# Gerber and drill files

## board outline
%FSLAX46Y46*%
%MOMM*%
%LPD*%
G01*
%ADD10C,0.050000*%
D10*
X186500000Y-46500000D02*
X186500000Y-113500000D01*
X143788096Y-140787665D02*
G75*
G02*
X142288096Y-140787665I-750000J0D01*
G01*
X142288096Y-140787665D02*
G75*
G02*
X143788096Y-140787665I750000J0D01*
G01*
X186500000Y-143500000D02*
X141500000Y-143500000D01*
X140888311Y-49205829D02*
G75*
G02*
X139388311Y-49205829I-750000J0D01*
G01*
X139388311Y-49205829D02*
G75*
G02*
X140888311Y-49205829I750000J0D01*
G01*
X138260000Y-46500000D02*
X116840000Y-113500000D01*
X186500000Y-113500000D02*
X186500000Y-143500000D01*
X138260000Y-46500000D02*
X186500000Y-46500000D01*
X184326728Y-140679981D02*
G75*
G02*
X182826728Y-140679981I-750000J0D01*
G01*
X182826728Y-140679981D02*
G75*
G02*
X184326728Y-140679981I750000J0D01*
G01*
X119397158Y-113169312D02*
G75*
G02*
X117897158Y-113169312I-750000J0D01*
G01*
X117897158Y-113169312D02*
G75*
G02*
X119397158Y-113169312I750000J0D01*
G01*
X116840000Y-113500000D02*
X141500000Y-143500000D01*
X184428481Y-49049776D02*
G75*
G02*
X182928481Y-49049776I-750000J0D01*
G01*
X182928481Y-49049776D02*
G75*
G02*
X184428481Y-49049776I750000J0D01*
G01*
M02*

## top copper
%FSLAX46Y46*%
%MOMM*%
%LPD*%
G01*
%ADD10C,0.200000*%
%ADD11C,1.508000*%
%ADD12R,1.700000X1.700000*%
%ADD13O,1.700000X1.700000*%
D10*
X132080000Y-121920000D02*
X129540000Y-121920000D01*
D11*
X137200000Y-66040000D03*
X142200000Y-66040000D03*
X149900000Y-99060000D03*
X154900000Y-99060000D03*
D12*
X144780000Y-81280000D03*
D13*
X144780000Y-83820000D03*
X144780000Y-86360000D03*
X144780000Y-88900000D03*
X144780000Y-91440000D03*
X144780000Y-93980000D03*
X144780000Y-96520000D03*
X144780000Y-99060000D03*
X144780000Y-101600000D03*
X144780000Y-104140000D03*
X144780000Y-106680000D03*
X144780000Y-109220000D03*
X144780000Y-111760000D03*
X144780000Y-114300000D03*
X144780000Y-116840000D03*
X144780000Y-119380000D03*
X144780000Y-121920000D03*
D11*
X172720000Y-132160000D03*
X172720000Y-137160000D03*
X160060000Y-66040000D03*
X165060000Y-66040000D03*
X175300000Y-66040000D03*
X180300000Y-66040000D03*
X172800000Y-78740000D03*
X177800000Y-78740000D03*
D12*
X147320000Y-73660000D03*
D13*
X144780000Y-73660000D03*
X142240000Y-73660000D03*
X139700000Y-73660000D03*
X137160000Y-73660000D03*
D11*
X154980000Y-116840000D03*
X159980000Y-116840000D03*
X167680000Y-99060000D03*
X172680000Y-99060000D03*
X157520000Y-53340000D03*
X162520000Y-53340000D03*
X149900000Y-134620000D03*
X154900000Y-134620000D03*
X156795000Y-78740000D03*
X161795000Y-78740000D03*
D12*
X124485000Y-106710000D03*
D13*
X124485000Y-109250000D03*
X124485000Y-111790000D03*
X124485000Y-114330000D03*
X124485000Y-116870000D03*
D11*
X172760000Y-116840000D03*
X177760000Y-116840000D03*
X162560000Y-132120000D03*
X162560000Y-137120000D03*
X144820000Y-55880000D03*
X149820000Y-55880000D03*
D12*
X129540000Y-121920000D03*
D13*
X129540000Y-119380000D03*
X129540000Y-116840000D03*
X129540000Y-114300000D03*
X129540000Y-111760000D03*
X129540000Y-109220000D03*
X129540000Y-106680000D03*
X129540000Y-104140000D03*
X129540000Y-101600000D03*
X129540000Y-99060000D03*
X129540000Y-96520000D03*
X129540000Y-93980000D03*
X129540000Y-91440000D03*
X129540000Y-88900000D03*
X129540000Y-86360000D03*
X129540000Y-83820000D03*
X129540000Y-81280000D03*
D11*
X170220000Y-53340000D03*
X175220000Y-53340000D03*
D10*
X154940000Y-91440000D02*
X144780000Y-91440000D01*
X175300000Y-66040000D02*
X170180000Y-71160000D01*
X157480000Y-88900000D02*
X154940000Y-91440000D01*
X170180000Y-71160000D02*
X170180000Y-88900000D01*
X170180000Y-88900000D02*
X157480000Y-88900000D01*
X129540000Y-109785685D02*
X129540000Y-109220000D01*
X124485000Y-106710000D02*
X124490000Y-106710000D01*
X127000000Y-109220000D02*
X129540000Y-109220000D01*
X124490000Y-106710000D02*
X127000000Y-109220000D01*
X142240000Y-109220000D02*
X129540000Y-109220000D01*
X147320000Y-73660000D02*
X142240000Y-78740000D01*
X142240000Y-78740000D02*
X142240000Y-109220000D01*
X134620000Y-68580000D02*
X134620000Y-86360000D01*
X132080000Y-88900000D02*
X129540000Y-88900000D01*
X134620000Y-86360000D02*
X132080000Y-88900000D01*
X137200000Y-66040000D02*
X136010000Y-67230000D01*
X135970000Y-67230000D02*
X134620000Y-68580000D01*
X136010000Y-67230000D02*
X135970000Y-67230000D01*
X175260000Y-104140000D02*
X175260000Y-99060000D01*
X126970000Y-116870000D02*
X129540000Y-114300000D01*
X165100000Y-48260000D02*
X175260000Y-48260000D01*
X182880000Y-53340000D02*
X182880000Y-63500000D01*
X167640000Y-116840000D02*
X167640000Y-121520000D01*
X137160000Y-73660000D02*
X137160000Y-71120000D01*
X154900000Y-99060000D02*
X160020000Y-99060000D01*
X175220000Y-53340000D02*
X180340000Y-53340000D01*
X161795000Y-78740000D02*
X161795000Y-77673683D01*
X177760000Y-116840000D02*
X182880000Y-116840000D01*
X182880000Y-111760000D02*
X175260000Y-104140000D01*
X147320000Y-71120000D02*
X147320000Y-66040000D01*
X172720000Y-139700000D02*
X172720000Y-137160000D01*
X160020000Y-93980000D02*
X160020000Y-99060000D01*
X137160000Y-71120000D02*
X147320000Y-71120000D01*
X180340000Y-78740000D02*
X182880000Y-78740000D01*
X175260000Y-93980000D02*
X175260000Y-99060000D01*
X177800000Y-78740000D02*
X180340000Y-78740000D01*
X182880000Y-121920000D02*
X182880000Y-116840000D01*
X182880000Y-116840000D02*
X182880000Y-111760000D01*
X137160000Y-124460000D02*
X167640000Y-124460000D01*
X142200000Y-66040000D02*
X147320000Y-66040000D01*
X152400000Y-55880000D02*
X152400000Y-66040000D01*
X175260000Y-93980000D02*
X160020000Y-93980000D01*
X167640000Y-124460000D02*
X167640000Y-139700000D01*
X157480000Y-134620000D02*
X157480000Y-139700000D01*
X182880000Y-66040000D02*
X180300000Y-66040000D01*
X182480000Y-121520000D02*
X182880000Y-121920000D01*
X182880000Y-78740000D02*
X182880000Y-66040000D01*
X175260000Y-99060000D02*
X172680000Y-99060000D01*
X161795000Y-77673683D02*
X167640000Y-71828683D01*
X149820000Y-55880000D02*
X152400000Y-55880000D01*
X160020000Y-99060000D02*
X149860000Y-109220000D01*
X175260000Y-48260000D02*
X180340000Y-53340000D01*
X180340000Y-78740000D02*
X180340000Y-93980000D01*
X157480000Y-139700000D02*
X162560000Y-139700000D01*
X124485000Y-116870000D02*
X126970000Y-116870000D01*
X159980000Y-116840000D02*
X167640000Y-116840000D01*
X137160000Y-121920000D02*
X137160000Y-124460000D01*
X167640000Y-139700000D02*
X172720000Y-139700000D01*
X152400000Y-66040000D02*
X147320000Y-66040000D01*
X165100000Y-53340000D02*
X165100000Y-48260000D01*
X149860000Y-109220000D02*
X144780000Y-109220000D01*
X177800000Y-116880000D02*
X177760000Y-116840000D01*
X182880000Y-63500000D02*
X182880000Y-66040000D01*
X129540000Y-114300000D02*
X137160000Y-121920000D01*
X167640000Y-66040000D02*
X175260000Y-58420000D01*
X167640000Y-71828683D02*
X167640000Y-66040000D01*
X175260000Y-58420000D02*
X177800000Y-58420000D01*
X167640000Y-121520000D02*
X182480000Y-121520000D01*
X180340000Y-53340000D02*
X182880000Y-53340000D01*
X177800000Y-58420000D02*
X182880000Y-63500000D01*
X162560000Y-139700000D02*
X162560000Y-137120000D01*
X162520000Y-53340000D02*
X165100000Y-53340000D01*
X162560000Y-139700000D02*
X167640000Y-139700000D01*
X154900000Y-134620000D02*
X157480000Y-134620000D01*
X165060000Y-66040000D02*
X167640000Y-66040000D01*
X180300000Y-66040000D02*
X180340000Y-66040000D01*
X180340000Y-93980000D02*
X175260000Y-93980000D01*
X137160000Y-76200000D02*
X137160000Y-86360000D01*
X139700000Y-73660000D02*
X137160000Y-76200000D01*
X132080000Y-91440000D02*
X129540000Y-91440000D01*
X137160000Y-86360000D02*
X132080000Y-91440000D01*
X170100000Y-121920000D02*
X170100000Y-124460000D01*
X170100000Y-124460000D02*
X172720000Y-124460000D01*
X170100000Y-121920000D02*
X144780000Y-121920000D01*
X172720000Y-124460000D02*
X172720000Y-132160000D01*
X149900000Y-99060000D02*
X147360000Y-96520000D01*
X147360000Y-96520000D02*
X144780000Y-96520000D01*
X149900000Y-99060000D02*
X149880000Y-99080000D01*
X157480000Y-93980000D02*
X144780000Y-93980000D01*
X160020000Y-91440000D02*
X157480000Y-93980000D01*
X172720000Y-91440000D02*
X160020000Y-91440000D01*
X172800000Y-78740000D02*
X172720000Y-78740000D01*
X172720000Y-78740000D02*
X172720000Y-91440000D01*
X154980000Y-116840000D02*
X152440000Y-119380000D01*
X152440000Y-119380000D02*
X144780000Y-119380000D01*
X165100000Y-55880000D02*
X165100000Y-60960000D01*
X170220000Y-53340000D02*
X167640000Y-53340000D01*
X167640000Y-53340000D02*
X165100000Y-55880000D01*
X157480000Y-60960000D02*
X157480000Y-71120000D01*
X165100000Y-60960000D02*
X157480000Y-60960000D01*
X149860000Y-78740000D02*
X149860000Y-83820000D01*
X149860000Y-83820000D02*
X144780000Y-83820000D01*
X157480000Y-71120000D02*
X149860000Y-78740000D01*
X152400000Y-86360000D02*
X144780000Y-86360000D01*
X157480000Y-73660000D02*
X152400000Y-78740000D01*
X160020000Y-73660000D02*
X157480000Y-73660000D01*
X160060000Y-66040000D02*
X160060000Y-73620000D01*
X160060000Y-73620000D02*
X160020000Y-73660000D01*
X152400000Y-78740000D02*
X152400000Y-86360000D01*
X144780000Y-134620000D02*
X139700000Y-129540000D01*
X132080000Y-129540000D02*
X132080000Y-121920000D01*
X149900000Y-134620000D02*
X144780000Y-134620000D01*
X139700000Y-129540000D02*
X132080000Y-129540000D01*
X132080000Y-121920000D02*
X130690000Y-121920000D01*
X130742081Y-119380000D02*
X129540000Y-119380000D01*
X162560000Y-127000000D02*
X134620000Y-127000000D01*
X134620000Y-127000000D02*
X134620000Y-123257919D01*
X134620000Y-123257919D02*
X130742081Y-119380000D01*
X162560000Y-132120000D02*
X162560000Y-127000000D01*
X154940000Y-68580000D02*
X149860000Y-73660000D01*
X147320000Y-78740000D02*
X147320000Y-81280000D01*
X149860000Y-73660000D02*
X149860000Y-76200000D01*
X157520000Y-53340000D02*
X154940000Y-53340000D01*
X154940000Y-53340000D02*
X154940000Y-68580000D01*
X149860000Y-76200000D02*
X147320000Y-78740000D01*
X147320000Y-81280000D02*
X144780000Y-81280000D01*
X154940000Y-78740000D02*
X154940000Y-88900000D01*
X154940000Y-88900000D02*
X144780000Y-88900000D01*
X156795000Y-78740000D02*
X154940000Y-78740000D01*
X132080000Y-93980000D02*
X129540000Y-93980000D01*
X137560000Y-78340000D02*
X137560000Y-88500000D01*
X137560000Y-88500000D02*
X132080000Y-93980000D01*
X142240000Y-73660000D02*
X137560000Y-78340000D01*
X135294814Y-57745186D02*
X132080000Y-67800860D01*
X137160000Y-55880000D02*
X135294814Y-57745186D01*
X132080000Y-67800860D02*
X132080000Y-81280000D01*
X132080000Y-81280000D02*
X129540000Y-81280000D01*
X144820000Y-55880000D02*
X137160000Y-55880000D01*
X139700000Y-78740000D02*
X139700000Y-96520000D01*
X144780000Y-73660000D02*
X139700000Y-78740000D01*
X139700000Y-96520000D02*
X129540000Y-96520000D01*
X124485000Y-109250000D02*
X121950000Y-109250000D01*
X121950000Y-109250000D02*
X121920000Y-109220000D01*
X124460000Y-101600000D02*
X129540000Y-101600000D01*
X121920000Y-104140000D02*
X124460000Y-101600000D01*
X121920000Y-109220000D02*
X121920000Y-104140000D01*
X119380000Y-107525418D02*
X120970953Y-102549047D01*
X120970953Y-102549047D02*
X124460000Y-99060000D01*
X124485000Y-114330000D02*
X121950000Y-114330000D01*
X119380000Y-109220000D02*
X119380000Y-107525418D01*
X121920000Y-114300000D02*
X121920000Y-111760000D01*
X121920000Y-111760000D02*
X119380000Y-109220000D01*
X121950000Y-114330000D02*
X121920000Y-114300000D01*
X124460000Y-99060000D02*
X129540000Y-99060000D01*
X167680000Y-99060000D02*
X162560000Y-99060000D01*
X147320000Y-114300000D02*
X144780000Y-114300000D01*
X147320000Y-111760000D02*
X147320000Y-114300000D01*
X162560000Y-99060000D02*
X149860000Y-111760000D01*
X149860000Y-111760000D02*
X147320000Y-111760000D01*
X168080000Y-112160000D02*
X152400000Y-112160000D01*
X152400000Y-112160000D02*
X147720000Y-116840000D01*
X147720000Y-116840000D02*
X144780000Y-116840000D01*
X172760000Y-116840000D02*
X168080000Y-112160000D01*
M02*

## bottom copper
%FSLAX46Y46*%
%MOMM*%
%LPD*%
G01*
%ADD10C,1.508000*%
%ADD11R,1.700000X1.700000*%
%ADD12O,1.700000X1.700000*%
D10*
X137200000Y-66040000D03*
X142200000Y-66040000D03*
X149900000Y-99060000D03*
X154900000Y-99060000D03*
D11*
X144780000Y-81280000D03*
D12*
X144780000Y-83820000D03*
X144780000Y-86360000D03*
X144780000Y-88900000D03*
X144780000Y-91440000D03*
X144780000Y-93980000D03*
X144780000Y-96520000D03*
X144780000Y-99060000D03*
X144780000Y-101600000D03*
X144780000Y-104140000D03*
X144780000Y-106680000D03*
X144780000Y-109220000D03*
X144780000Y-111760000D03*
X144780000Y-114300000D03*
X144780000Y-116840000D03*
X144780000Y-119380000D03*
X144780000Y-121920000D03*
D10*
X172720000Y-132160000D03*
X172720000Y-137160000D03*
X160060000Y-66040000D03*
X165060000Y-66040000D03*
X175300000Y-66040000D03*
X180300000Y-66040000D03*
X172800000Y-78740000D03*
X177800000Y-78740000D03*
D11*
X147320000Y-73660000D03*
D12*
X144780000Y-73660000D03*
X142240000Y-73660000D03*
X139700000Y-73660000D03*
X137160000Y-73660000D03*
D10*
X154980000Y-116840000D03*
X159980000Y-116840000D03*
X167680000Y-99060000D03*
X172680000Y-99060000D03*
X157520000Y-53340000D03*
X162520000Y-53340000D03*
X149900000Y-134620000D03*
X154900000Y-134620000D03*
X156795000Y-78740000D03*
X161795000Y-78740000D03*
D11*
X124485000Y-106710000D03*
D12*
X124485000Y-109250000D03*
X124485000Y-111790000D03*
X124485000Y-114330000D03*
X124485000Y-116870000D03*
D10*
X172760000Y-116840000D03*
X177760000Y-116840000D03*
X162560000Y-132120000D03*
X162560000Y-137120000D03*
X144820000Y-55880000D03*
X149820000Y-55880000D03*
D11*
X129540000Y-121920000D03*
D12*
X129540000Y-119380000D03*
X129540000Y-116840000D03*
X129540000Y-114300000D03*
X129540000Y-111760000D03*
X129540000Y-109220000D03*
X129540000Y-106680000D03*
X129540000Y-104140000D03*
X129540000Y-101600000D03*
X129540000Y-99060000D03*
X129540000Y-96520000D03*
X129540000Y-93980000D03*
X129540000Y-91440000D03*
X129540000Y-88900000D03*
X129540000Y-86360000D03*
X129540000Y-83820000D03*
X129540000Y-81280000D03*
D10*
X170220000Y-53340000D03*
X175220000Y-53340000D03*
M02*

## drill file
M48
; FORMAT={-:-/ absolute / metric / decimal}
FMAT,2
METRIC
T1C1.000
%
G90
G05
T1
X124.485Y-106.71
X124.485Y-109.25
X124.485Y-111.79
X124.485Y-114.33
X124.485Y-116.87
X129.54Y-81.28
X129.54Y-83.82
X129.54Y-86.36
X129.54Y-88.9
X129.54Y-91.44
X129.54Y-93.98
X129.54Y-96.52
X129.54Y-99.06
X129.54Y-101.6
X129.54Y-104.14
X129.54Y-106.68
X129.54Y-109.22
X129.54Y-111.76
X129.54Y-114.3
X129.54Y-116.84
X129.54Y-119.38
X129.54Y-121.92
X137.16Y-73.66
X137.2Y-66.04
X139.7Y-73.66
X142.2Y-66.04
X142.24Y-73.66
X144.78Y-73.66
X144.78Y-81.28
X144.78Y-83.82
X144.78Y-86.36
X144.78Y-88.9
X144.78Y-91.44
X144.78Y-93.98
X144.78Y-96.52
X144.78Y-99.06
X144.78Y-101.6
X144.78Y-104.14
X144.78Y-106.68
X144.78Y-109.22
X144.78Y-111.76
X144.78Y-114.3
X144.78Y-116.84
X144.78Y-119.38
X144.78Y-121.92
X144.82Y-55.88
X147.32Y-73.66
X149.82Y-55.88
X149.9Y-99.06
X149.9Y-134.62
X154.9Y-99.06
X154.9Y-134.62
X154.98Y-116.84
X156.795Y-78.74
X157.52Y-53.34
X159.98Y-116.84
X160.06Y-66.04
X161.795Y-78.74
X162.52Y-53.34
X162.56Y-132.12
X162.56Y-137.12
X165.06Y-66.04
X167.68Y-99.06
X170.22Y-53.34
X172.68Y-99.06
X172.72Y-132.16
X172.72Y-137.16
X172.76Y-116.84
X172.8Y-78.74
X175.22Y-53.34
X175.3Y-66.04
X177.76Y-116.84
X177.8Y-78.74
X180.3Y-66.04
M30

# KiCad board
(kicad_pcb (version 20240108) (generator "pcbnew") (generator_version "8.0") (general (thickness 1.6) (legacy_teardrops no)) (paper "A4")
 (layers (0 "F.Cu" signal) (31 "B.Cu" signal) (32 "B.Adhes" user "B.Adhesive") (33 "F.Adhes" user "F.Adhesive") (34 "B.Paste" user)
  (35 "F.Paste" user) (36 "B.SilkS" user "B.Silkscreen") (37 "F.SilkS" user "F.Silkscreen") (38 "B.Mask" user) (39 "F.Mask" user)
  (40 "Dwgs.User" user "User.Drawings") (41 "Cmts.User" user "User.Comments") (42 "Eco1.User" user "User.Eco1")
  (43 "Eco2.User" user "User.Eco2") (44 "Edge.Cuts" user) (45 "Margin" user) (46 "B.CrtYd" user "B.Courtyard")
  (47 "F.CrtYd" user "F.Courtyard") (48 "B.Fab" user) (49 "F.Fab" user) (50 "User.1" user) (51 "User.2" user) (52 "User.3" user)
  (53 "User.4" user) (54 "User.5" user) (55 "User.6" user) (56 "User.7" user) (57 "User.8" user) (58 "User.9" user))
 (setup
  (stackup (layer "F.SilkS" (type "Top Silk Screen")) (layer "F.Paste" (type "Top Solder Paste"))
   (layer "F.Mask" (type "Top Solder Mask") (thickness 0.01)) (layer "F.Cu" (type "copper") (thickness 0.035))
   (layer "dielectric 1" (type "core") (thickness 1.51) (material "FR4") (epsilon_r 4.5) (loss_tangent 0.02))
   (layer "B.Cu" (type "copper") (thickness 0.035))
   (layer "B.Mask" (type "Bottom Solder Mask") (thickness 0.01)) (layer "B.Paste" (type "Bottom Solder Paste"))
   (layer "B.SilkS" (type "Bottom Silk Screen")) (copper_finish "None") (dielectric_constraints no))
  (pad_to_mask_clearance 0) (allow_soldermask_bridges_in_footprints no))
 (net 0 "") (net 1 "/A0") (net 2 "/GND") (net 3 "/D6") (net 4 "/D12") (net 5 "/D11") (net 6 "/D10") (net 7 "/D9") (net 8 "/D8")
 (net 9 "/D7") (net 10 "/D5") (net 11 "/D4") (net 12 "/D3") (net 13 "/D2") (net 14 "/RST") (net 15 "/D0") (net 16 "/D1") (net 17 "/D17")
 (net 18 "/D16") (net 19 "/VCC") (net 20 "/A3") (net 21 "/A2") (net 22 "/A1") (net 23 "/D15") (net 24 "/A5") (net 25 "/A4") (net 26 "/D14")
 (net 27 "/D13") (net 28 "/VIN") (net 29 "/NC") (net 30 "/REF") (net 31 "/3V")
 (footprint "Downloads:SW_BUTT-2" (layer "F.Cu") (at 139.7 66.04)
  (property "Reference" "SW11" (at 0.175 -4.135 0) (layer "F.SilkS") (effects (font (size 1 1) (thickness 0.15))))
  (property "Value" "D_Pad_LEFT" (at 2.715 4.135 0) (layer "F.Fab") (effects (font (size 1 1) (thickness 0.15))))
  (pad "1" thru_hole circle (at -2.5 0) (size 1.508 1.508) (drill 1) (layers "*.Cu" "*.Mask") (remove_unused_layers no) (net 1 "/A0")
   (solder_mask_margin 0.102))
  (pad "2" thru_hole circle (at 2.5 0) (size 1.508 1.508) (drill 1) (layers "*.Cu" "*.Mask") (remove_unused_layers no) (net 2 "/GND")
   (solder_mask_margin 0.102)))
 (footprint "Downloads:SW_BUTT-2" (layer "F.Cu") (at 152.4 99.06)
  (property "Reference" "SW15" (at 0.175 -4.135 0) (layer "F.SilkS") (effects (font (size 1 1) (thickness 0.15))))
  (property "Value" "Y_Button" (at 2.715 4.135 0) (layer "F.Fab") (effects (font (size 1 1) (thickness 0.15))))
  (pad "1" thru_hole circle (at -2.5 0) (size 1.508 1.508) (drill 1) (layers "*.Cu" "*.Mask") (remove_unused_layers no) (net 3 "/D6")
   (solder_mask_margin 0.102))
  (pad "2" thru_hole circle (at 2.5 0) (size 1.508 1.508) (drill 1) (layers "*.Cu" "*.Mask") (remove_unused_layers no) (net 2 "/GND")
   (solder_mask_margin 0.102)))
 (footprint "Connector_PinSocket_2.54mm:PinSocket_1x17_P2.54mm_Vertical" (layer "F.Cu") (at 144.78 81.28)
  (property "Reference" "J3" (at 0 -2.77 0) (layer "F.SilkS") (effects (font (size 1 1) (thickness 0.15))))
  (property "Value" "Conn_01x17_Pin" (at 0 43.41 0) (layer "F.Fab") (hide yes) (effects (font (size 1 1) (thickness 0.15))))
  (pad "1" thru_hole rect (at 0 0) (size 1.7 1.7) (drill 1) (layers "*.Cu" "*.Mask") (remove_unused_layers no) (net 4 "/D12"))
  (pad "2" thru_hole oval (at 0 2.54) (size 1.7 1.7) (drill 1) (layers "*.Cu" "*.Mask") (remove_unused_layers no) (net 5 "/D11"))
  (pad "3" thru_hole oval (at 0 5.08) (size 1.7 1.7) (drill 1) (layers "*.Cu" "*.Mask") (remove_unused_layers no) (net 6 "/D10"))
  (pad "4" thru_hole oval (at 0 7.62) (size 1.7 1.7) (drill 1) (layers "*.Cu" "*.Mask") (remove_unused_layers no) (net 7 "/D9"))
  (pad "5" thru_hole oval (at 0 10.16) (size 1.7 1.7) (drill 1) (layers "*.Cu" "*.Mask") (remove_unused_layers no) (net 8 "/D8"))
  (pad "6" thru_hole oval (at 0 12.7) (size 1.7 1.7) (drill 1) (layers "*.Cu" "*.Mask") (remove_unused_layers no) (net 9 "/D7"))
  (pad "7" thru_hole oval (at 0 15.24) (size 1.7 1.7) (drill 1) (layers "*.Cu" "*.Mask") (remove_unused_layers no) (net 3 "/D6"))
  (pad "8" thru_hole oval (at 0 17.78) (size 1.7 1.7) (drill 1) (layers "*.Cu" "*.Mask") (remove_unused_layers no) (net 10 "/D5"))
  (pad "9" thru_hole oval (at 0 20.32) (size 1.7 1.7) (drill 1) (layers "*.Cu" "*.Mask") (remove_unused_layers no) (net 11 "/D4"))
  (pad "10" thru_hole oval (at 0 22.86) (size 1.7 1.7) (drill 1) (layers "*.Cu" "*.Mask") (remove_unused_layers no) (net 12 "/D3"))
  (pad "11" thru_hole oval (at 0 25.4) (size 1.7 1.7) (drill 1) (layers "*.Cu" "*.Mask") (remove_unused_layers no) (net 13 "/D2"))
  (pad "12" thru_hole oval (at 0 27.94) (size 1.7 1.7) (drill 1) (layers "*.Cu" "*.Mask") (remove_unused_layers no) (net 2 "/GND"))
  (pad "13" thru_hole oval (at 0 30.48) (size 1.7 1.7) (drill 1) (layers "*.Cu" "*.Mask") (remove_unused_layers no) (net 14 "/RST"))
  (pad "14" thru_hole oval (at 0 33.02) (size 1.7 1.7) (drill 1) (layers "*.Cu" "*.Mask") (remove_unused_layers no) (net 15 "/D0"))
  (pad "15" thru_hole oval (at 0 35.56) (size 1.7 1.7) (drill 1) (layers "*.Cu" "*.Mask") (remove_unused_layers no) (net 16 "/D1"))
  (pad "16" thru_hole oval (at 0 38.1) (size 1.7 1.7) (drill 1) (layers "*.Cu" "*.Mask") (remove_unused_layers no) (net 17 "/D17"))
  (pad "17" thru_hole oval (at 0 40.64) (size 1.7 1.7) (drill 1) (layers "*.Cu" "*.Mask") (remove_unused_layers no) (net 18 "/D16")))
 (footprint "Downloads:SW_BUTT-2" (layer "F.Cu") (at 172.72 134.66 -90)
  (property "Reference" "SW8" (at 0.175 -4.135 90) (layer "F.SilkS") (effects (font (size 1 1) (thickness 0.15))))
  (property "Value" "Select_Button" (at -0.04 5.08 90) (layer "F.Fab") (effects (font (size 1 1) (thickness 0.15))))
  (pad "1" thru_hole circle (at -2.5 0 270) (size 1.508 1.508) (drill 1) (layers "*.Cu" "*.Mask") (remove_unused_layers no) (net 18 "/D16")
   (solder_mask_margin 0.102))
  (pad "2" thru_hole circle (at 2.5 0 270) (size 1.508 1.508) (drill 1) (layers "*.Cu" "*.Mask") (remove_unused_layers no) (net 2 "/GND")
   (solder_mask_margin 0.102)))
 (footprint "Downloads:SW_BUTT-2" (layer "F.Cu") (at 162.56 66.04)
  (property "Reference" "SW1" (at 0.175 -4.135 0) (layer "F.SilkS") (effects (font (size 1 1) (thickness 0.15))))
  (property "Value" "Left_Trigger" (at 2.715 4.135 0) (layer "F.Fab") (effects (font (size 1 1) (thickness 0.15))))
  (pad "1" thru_hole circle (at -2.5 0) (size 1.508 1.508) (drill 1) (layers "*.Cu" "*.Mask") (remove_unused_layers no) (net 6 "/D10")
   (solder_mask_margin 0.102))
  (pad "2" thru_hole circle (at 2.5 0) (size 1.508 1.508) (drill 1) (layers "*.Cu" "*.Mask") (remove_unused_layers no) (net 2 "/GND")
   (solder_mask_margin 0.102)))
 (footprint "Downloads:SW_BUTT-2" (layer "F.Cu") (at 177.8 66.04)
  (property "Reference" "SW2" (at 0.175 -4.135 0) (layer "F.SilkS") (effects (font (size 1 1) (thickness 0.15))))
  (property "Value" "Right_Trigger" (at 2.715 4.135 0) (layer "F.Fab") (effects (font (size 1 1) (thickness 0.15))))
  (pad "1" thru_hole circle (at -2.5 0) (size 1.508 1.508) (drill 1) (layers "*.Cu" "*.Mask") (remove_unused_layers no) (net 8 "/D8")
   (solder_mask_margin 0.102))
  (pad "2" thru_hole circle (at 2.5 0) (size 1.508 1.508) (drill 1) (layers "*.Cu" "*.Mask") (remove_unused_layers no) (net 2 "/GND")
   (solder_mask_margin 0.102)))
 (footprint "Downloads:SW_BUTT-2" (layer "F.Cu") (at 175.3 78.74)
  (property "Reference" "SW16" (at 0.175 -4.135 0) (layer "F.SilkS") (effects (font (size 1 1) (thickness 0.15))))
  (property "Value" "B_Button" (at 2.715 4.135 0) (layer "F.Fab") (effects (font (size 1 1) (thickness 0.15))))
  (pad "1" thru_hole circle (at -2.5 0) (size 1.508 1.508) (drill 1) (layers "*.Cu" "*.Mask") (remove_unused_layers no) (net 9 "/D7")
   (solder_mask_margin 0.102))
  (pad "2" thru_hole circle (at 2.5 0) (size 1.508 1.508) (drill 1) (layers "*.Cu" "*.Mask") (remove_unused_layers no) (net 2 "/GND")
   (solder_mask_margin 0.102)))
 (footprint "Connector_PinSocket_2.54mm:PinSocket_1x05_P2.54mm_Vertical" (layer "F.Cu") (at 147.32 73.66 -90)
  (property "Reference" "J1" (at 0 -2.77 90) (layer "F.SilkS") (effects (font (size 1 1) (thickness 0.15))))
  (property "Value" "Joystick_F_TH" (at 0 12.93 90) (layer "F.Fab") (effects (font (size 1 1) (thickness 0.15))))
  (pad "1" thru_hole rect (at 0 0 270) (size 1.7 1.7) (drill 1) (layers "*.Cu" "*.Mask") (remove_unused_layers no) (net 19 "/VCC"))
  (pad "2" thru_hole oval (at 0 2.54 270) (size 1.7 1.7) (drill 1) (layers "*.Cu" "*.Mask") (remove_unused_layers no) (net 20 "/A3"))
  (pad "3" thru_hole oval (at 0 5.08 270) (size 1.7 1.7) (drill 1) (layers "*.Cu" "*.Mask") (remove_unused_layers no) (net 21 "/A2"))
  (pad "4" thru_hole oval (at 0 7.62 270) (size 1.7 1.7) (drill 1) (layers "*.Cu" "*.Mask") (remove_unused_layers no) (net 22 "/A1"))
  (pad "5" thru_hole oval (at 0 10.16 270) (size 1.7 1.7) (drill 1) (layers "*.Cu" "*.Mask") (remove_unused_layers no) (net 2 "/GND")))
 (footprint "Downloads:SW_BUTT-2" (layer "F.Cu") (at 157.48 116.84)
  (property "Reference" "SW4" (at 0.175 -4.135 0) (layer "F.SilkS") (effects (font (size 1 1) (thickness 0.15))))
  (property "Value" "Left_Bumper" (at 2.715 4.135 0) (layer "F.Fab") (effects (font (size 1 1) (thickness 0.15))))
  (pad "1" thru_hole circle (at -2.5 0) (size 1.508 1.508) (drill 1) (layers "*.Cu" "*.Mask") (remove_unused_layers no) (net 17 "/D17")
   (solder_mask_margin 0.102))
  (pad "2" thru_hole circle (at 2.5 0) (size 1.508 1.508) (drill 1) (layers "*.Cu" "*.Mask") (remove_unused_layers no) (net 2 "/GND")
   (solder_mask_margin 0.102)))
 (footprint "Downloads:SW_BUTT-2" (layer "F.Cu") (at 170.18 99.06)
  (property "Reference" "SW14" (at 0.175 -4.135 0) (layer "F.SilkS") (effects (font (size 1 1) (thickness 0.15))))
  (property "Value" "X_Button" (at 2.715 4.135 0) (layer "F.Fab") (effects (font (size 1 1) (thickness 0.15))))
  (pad "1" thru_hole circle (at -2.5 0) (size 1.508 1.508) (drill 1) (layers "*.Cu" "*.Mask") (remove_unused_layers no) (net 15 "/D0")
   (solder_mask_margin 0.102))
  (pad "2" thru_hole circle (at 2.5 0) (size 1.508 1.508) (drill 1) (layers "*.Cu" "*.Mask") (remove_unused_layers no) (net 2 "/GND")
   (solder_mask_margin 0.102)))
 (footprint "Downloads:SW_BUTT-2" (layer "F.Cu") (at 160.02 53.34)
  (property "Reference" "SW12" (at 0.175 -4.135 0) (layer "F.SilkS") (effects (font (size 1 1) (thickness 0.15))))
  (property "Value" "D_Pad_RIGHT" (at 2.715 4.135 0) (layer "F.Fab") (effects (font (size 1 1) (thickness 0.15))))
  (pad "1" thru_hole circle (at -2.5 0) (size 1.508 1.508) (drill 1) (layers "*.Cu" "*.Mask") (remove_unused_layers no) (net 4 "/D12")
   (solder_mask_margin 0.102))
  (pad "2" thru_hole circle (at 2.5 0) (size 1.508 1.508) (drill 1) (layers "*.Cu" "*.Mask") (remove_unused_layers no) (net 2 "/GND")
   (solder_mask_margin 0.102)))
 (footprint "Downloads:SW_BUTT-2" (layer "F.Cu") (at 152.4 134.62)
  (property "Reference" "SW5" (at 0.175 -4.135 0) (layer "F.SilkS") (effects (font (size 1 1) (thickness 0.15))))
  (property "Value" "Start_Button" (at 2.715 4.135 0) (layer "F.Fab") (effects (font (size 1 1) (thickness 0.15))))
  (pad "1" thru_hole circle (at -2.5 0) (size 1.508 1.508) (drill 1) (layers "*.Cu" "*.Mask") (remove_unused_layers no) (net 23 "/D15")
   (solder_mask_margin 0.102))
  (pad "2" thru_hole circle (at 2.5 0) (size 1.508 1.508) (drill 1) (layers "*.Cu" "*.Mask") (remove_unused_layers no) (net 2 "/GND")
   (solder_mask_margin 0.102)))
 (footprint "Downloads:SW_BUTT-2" (layer "F.Cu") (at 159.295 78.74)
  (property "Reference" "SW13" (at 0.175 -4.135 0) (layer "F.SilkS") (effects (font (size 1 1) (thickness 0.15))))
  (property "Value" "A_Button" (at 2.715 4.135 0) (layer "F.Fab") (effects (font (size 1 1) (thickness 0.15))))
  (pad "1" thru_hole circle (at -2.5 0) (size 1.508 1.508) (drill 1) (layers "*.Cu" "*.Mask") (remove_unused_layers no) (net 7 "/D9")
   (solder_mask_margin 0.102))
  (pad "2" thru_hole circle (at 2.5 0) (size 1.508 1.508) (drill 1) (layers "*.Cu" "*.Mask") (remove_unused_layers no) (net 2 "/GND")
   (solder_mask_margin 0.102)))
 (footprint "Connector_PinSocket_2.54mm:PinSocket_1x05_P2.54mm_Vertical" (layer "F.Cu") (at 124.485 106.71)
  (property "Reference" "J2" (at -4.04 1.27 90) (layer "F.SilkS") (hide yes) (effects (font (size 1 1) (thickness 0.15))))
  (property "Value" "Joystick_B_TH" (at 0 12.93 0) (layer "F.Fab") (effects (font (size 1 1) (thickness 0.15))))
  (pad "1" thru_hole rect (at 0 0) (size 1.7 1.7) (drill 1) (layers "*.Cu" "*.Mask") (remove_unused_layers no) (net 19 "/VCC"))
  (pad "2" thru_hole oval (at 0 2.54) (size 1.7 1.7) (drill 1) (layers "*.Cu" "*.Mask") (remove_unused_layers no) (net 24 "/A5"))
  (pad "3" thru_hole oval (at 0 5.08) (size 1.7 1.7) (drill 1) (layers "*.Cu" "*.Mask") (remove_unused_layers no) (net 9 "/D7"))
  (pad "4" thru_hole oval (at 0 7.62) (size 1.7 1.7) (drill 1) (layers "*.Cu" "*.Mask") (remove_unused_layers no) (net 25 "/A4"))
  (pad "5" thru_hole oval (at 0 10.16) (size 1.7 1.7) (drill 1) (layers "*.Cu" "*.Mask") (remove_unused_layers no) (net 2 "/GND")))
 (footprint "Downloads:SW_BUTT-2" (layer "F.Cu") (at 175.26 116.84)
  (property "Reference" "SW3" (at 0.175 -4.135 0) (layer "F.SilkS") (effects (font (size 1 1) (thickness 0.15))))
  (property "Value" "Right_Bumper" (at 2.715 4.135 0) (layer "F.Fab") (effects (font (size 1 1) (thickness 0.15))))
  (pad "1" thru_hole circle (at -2.5 0) (size 1.508 1.508) (drill 1) (layers "*.Cu" "*.Mask") (remove_unused_layers no) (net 16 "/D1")
   (solder_mask_margin 0.102))
  (pad "2" thru_hole circle (at 2.5 0) (size 1.508 1.508) (drill 1) (layers "*.Cu" "*.Mask") (remove_unused_layers no) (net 2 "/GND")
   (solder_mask_margin 0.102)))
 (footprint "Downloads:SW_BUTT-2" (layer "F.Cu") (at 162.56 134.62 -90)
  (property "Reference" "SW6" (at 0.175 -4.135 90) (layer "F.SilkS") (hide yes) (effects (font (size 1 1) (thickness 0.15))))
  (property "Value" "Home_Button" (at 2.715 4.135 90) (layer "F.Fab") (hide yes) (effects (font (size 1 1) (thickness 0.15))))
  (pad "1" thru_hole circle (at -2.5 0 270) (size 1.508 1.508) (drill 1) (layers "*.Cu" "*.Mask") (remove_unused_layers no) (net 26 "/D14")
   (solder_mask_margin 0.102))
  (pad "2" thru_hole circle (at 2.5 0 270) (size 1.508 1.508) (drill 1) (layers "*.Cu" "*.Mask") (remove_unused_layers no) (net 2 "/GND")
   (solder_mask_margin 0.102)))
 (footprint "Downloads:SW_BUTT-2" (layer "F.Cu") (at 147.32 55.88)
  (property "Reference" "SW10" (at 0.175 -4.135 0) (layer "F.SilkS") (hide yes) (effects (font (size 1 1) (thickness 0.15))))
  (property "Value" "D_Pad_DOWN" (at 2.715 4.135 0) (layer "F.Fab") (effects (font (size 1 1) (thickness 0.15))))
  (pad "1" thru_hole circle (at -2.5 0) (size 1.508 1.508) (drill 1) (layers "*.Cu" "*.Mask") (remove_unused_layers no) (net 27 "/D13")
   (solder_mask_margin 0.102))
  (pad "2" thru_hole circle (at 2.5 0) (size 1.508 1.508) (drill 1) (layers "*.Cu" "*.Mask") (remove_unused_layers no) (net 2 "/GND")
   (solder_mask_margin 0.102)))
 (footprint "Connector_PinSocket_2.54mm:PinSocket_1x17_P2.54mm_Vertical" (layer "F.Cu") (at 129.54 121.92 180)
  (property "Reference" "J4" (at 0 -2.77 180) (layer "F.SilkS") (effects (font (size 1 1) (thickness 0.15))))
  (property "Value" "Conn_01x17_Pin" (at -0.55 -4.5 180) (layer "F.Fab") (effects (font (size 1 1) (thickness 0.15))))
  (pad "1" thru_hole rect (at 0 0 180) (size 1.7 1.7) (drill 1) (layers "*.Cu" "*.Mask") (remove_unused_layers no) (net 23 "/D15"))
  (pad "2" thru_hole oval (at 0 2.54 180) (size 1.7 1.7) (drill 1) (layers "*.Cu" "*.Mask") (remove_unused_layers no) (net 26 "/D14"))
  (pad "3" thru_hole oval (at 0 5.08 180) (size 1.7 1.7) (drill 1) (layers "*.Cu" "*.Mask") (remove_unused_layers no) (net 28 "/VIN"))
  (pad "4" thru_hole oval (at 0 7.62 180) (size 1.7 1.7) (drill 1) (layers "*.Cu" "*.Mask") (remove_unused_layers no) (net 2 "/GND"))
  (pad "5" thru_hole oval (at 0 10.16 180) (size 1.7 1.7) (drill 1) (layers "*.Cu" "*.Mask") (remove_unused_layers no) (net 14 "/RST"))
  (pad "6" thru_hole oval (at 0 12.7 180) (size 1.7 1.7) (drill 1) (layers "*.Cu" "*.Mask") (remove_unused_layers no) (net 19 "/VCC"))
  (pad "7" thru_hole oval (at 0 15.24 180) (size 1.7 1.7) (drill 1) (layers "*.Cu" "*.Mask") (remove_unused_layers no) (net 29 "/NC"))
  (pad "8" thru_hole oval (at 0 17.78 180) (size 1.7 1.7) (drill 1) (layers "*.Cu" "*.Mask") (remove_unused_layers no) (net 29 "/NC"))
  (pad "9" thru_hole oval (at 0 20.32 180) (size 1.7 1.7) (drill 1) (layers "*.Cu" "*.Mask") (remove_unused_layers no) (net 24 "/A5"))
  (pad "10" thru_hole oval (at 0 22.86 180) (size 1.7 1.7) (drill 1) (layers "*.Cu" "*.Mask") (remove_unused_layers no) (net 25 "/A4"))
  (pad "11" thru_hole oval (at 0 25.4 180) (size 1.7 1.7) (drill 1) (layers "*.Cu" "*.Mask") (remove_unused_layers no) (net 20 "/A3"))
  (pad "12" thru_hole oval (at 0 27.94 180) (size 1.7 1.7) (drill 1) (layers "*.Cu" "*.Mask") (remove_unused_layers no) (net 21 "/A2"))
  (pad "13" thru_hole oval (at 0 30.48 180) (size 1.7 1.7) (drill 1) (layers "*.Cu" "*.Mask") (remove_unused_layers no) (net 22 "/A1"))
  (pad "14" thru_hole oval (at 0 33.02 180) (size 1.7 1.7) (drill 1) (layers "*.Cu" "*.Mask") (remove_unused_layers no) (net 1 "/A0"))
  (pad "15" thru_hole oval (at 0 35.56 180) (size 1.7 1.7) (drill 1) (layers "*.Cu" "*.Mask") (remove_unused_layers no) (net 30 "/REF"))
  (pad "16" thru_hole oval (at 0 38.1 180) (size 1.7 1.7) (drill 1) (layers "*.Cu" "*.Mask") (remove_unused_layers no) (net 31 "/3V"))
  (pad "17" thru_hole oval (at 0 40.64 180) (size 1.7 1.7) (drill 1) (layers "*.Cu" "*.Mask") (remove_unused_layers no) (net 27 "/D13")))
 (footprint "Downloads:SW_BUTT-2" (layer "F.Cu") (at 172.72 53.34)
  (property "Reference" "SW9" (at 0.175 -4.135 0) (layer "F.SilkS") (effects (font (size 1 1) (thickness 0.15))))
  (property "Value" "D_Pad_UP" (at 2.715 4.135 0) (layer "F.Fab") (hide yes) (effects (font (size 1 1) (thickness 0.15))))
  (pad "1" thru_hole circle (at -2.5 0) (size 1.508 1.508) (drill 1) (layers "*.Cu" "*.Mask") (remove_unused_layers no) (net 5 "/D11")
   (solder_mask_margin 0.102))
  (pad "2" thru_hole circle (at 2.5 0) (size 1.508 1.508) (drill 1) (layers "*.Cu" "*.Mask") (remove_unused_layers no) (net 2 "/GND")
   (solder_mask_margin 0.102)))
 (gr_line (start 132.08 121.92) (end 129.54 121.92) (stroke (width 0.2) (type default)) (layer "F.Cu") (net 23))
 (gr_line (start 186.5 46.5) (end 186.5 113.5) (stroke (width 0.05) (type default)) (layer "Edge.Cuts"))
 (gr_circle (center 143.038096 140.787665) (end 143.788096 140.787665) (stroke (width 0.05) (type default)) (fill none) (layer "Edge.Cuts"))
 (gr_line (start 186.5 143.5) (end 141.5 143.5) (stroke (width 0.05) (type default)) (layer "Edge.Cuts"))
 (gr_circle (center 140.138311 49.205829) (end 140.888311 49.205829) (stroke (width 0.05) (type default)) (fill none) (layer "Edge.Cuts"))
 (gr_line (start 138.26 46.5) (end 116.84 113.5) (stroke (width 0.05) (type default)) (layer "Edge.Cuts"))
 (gr_line (start 186.5 113.5) (end 186.5 143.5) (stroke (width 0.05) (type default)) (layer "Edge.Cuts"))
 (gr_line (start 138.26 46.5) (end 186.5 46.5) (stroke (width 0.05) (type default)) (layer "Edge.Cuts"))
 (gr_circle (center 183.576728 140.679981) (end 184.326728 140.679981) (stroke (width 0.05) (type default)) (fill none) (layer "Edge.Cuts"))
 (gr_circle (center 118.647158 113.169312) (end 119.397158 113.169312) (stroke (width 0.05) (type default)) (fill none) (layer "Edge.Cuts"))
 (gr_line (start 116.84 113.5) (end 141.5 143.5) (stroke (width 0.05) (type default)) (layer "Edge.Cuts"))
 (gr_circle (center 183.678481 49.049776) (end 184.428481 49.049776) (stroke (width 0.05) (type default)) (fill none) (layer "Edge.Cuts"))
 (segment (start 154.94 91.44) (end 144.78 91.44) (width 0.2) (layer "F.Cu") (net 8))
 (segment (start 175.3 66.04) (end 170.18 71.16) (width 0.2) (layer "F.Cu") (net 8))
 (segment (start 157.48 88.9) (end 154.94 91.44) (width 0.2) (layer "F.Cu") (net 8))
 (segment (start 170.18 71.16) (end 170.18 88.9) (width 0.2) (layer "F.Cu") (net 8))
 (segment (start 170.18 88.9) (end 157.48 88.9) (width 0.2) (layer "F.Cu") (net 8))
 (segment (start 129.54 109.785685) (end 129.54 109.22) (width 0.2) (layer "F.Cu") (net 19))
 (segment (start 124.485 106.71) (end 124.49 106.71) (width 0.2) (layer "F.Cu") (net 19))
 (segment (start 127 109.22) (end 129.54 109.22) (width 0.2) (layer "F.Cu") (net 19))
 (segment (start 124.49 106.71) (end 127 109.22) (width 0.2) (layer "F.Cu") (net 19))
 (segment (start 142.24 109.22) (end 129.54 109.22) (width 0.2) (layer "F.Cu") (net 19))
 (segment (start 147.32 73.66) (end 142.24 78.74) (width 0.2) (layer "F.Cu") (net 19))
 (segment (start 142.24 78.74) (end 142.24 109.22) (width 0.2) (layer "F.Cu") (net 19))
 (segment (start 134.62 68.58) (end 134.62 86.36) (width 0.2) (layer "F.Cu") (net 1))
 (segment (start 132.08 88.9) (end 129.54 88.9) (width 0.2) (layer "F.Cu") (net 1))
 (segment (start 134.62 86.36) (end 132.08 88.9) (width 0.2) (layer "F.Cu") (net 1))
 (segment (start 137.2 66.04) (end 136.01 67.23) (width 0.2) (layer "F.Cu") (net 1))
 (segment (start 135.97 67.23) (end 134.62 68.58) (width 0.2) (layer "F.Cu") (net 1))
 (segment (start 136.01 67.23) (end 135.97 67.23) (width 0.2) (layer "F.Cu") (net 1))
 (segment (start 175.26 104.14) (end 175.26 99.06) (width 0.2) (layer "F.Cu") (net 2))
 (segment (start 126.97 116.87) (end 129.54 114.3) (width 0.2) (layer "F.Cu") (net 2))
 (segment (start 165.1 48.26) (end 175.26 48.26) (width 0.2) (layer "F.Cu") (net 2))
 (segment (start 182.88 53.34) (end 182.88 63.5) (width 0.2) (layer "F.Cu") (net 2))
 (segment (start 167.64 116.84) (end 167.64 121.52) (width 0.2) (layer "F.Cu") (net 2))
 (segment (start 137.16 73.66) (end 137.16 71.12) (width 0.2) (layer "F.Cu") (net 2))
 (segment (start 154.9 99.06) (end 160.02 99.06) (width 0.2) (layer "F.Cu") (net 2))
 (segment (start 175.22 53.34) (end 180.34 53.34) (width 0.2) (layer "F.Cu") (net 2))
 (segment (start 161.795 78.74) (end 161.795 77.673683) (width 0.2) (layer "F.Cu") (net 2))
 (segment (start 177.76 116.84) (end 182.88 116.84) (width 0.2) (layer "F.Cu") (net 2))
 (segment (start 182.88 111.76) (end 175.26 104.14) (width 0.2) (layer "F.Cu") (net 2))
 (segment (start 147.32 71.12) (end 147.32 66.04) (width 0.2) (layer "F.Cu") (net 2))
 (segment (start 172.72 139.7) (end 172.72 137.16) (width 0.2) (layer "F.Cu") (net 2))
 (segment (start 160.02 93.98) (end 160.02 99.06) (width 0.2) (layer "F.Cu") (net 2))
 (segment (start 137.16 71.12) (end 147.32 71.12) (width 0.2) (layer "F.Cu") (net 2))
 (segment (start 180.34 78.74) (end 182.88 78.74) (width 0.2) (layer "F.Cu") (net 2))
 (segment (start 175.26 93.98) (end 175.26 99.06) (width 0.2) (layer "F.Cu") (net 2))
 (segment (start 177.8 78.74) (end 180.34 78.74) (width 0.2) (layer "F.Cu") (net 2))
 (segment (start 182.88 121.92) (end 182.88 116.84) (width 0.2) (layer "F.Cu") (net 2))
 (segment (start 182.88 116.84) (end 182.88 111.76) (width 0.2) (layer "F.Cu") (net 2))
 (segment (start 137.16 124.46) (end 167.64 124.46) (width 0.2) (layer "F.Cu") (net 2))
 (segment (start 142.2 66.04) (end 147.32 66.04) (width 0.2) (layer "F.Cu") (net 2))
 (segment (start 152.4 55.88) (end 152.4 66.04) (width 0.2) (layer "F.Cu") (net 2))
 (segment (start 175.26 93.98) (end 160.02 93.98) (width 0.2) (layer "F.Cu") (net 2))
 (segment (start 167.64 124.46) (end 167.64 139.7) (width 0.2) (layer "F.Cu") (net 2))
 (segment (start 157.48 134.62) (end 157.48 139.7) (width 0.2) (layer "F.Cu") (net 2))
 (segment (start 182.88 66.04) (end 180.3 66.04) (width 0.2) (layer "F.Cu") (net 2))
 (segment (start 182.48 121.52) (end 182.88 121.92) (width 0.2) (layer "F.Cu") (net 2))
 (segment (start 182.88 78.74) (end 182.88 66.04) (width 0.2) (layer "F.Cu") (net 2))
 (segment (start 175.26 99.06) (end 172.68 99.06) (width 0.2) (layer "F.Cu") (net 2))
 (segment (start 161.795 77.673683) (end 167.64 71.828683) (width 0.2) (layer "F.Cu") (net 2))
 (segment (start 149.82 55.88) (end 152.4 55.88) (width 0.2) (layer "F.Cu") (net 2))
 (segment (start 160.02 99.06) (end 149.86 109.22) (width 0.2) (layer "F.Cu") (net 2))
 (segment (start 175.26 48.26) (end 180.34 53.34) (width 0.2) (layer "F.Cu") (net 2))
 (segment (start 180.34 78.74) (end 180.34 93.98) (width 0.2) (layer "F.Cu") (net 2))
 (segment (start 157.48 139.7) (end 162.56 139.7) (width 0.2) (layer "F.Cu") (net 2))
 (segment (start 124.485 116.87) (end 126.97 116.87) (width 0.2) (layer "F.Cu") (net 2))
 (segment (start 159.98 116.84) (end 167.64 116.84) (width 0.2) (layer "F.Cu") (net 2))
 (segment (start 137.16 121.92) (end 137.16 124.46) (width 0.2) (layer "F.Cu") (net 2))
 (segment (start 167.64 139.7) (end 172.72 139.7) (width 0.2) (layer "F.Cu") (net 2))
 (segment (start 152.4 66.04) (end 147.32 66.04) (width 0.2) (layer "F.Cu") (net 2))
 (segment (start 165.1 53.34) (end 165.1 48.26) (width 0.2) (layer "F.Cu") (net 2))
 (segment (start 149.86 109.22) (end 144.78 109.22) (width 0.2) (layer "F.Cu") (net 2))
 (segment (start 177.8 116.88) (end 177.76 116.84) (width 0.2) (layer "F.Cu") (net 2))
 (segment (start 182.88 63.5) (end 182.88 66.04) (width 0.2) (layer "F.Cu") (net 2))
 (segment (start 129.54 114.3) (end 137.16 121.92) (width 0.2) (layer "F.Cu") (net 2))
 (segment (start 167.64 66.04) (end 175.26 58.42) (width 0.2) (layer "F.Cu") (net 2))
 (segment (start 167.64 71.828683) (end 167.64 66.04) (width 0.2) (layer "F.Cu") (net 2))
 (segment (start 175.26 58.42) (end 177.8 58.42) (width 0.2) (layer "F.Cu") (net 2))
 (segment (start 167.64 121.52) (end 182.48 121.52) (width 0.2) (layer "F.Cu") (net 2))
 (segment (start 180.34 53.34) (end 182.88 53.34) (width 0.2) (layer "F.Cu") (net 2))
 (segment (start 177.8 58.42) (end 182.88 63.5) (width 0.2) (layer "F.Cu") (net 2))
 (segment (start 162.56 139.7) (end 162.56 137.12) (width 0.2) (layer "F.Cu") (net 2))
 (segment (start 162.52 53.34) (end 165.1 53.34) (width 0.2) (layer "F.Cu") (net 2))
 (segment (start 162.56 139.7) (end 167.64 139.7) (width 0.2) (layer "F.Cu") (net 2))
 (segment (start 154.9 134.62) (end 157.48 134.62) (width 0.2) (layer "F.Cu") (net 2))
 (segment (start 165.06 66.04) (end 167.64 66.04) (width 0.2) (layer "F.Cu") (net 2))
 (segment (start 180.3 66.04) (end 180.34 66.04) (width 0.2) (layer "F.Cu") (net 2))
 (segment (start 180.34 93.98) (end 175.26 93.98) (width 0.2) (layer "F.Cu") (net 2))
 (segment (start 137.16 76.2) (end 137.16 86.36) (width 0.2) (layer "F.Cu") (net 22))
 (segment (start 139.7 73.66) (end 137.16 76.2) (width 0.2) (layer "F.Cu") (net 22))
 (segment (start 132.08 91.44) (end 129.54 91.44) (width 0.2) (layer "F.Cu") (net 22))
 (segment (start 137.16 86.36) (end 132.08 91.44) (width 0.2) (layer "F.Cu") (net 22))
 (segment (start 170.1 121.92) (end 170.1 124.46) (width 0.2) (layer "F.Cu") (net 18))
 (segment (start 170.1 124.46) (end 172.72 124.46) (width 0.2) (layer "F.Cu") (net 18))
 (segment (start 170.1 121.92) (end 144.78 121.92) (width 0.2) (layer "F.Cu") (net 18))
 (segment (start 172.72 124.46) (end 172.72 132.16) (width 0.2) (layer "F.Cu") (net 18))
 (segment (start 149.9 99.06) (end 147.36 96.52) (width 0.2) (layer "F.Cu") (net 3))
 (segment (start 147.36 96.52) (end 144.78 96.52) (width 0.2) (layer "F.Cu") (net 3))
 (segment (start 149.9 99.06) (end 149.88 99.08) (width 0.2) (layer "F.Cu") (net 3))
 (segment (start 157.48 93.98) (end 144.78 93.98) (width 0.2) (layer "F.Cu") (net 9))
 (segment (start 160.02 91.44) (end 157.48 93.98) (width 0.2) (layer "F.Cu") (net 9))
 (segment (start 172.72 91.44) (end 160.02 91.44) (width 0.2) (layer "F.Cu") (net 9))
 (segment (start 172.8 78.74) (end 172.72 78.74) (width 0.2) (layer "F.Cu") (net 9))
 (segment (start 172.72 78.74) (end 172.72 91.44) (width 0.2) (layer "F.Cu") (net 9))
 (segment (start 154.98 116.84) (end 152.44 119.38) (width 0.2) (layer "F.Cu") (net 17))
 (segment (start 152.44 119.38) (end 144.78 119.38) (width 0.2) (layer "F.Cu") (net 17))
 (segment (start 165.1 55.88) (end 165.1 60.96) (width 0.2) (layer "F.Cu") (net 5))
 (segment (start 170.22 53.34) (end 167.64 53.34) (width 0.2) (layer "F.Cu") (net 5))
 (segment (start 167.64 53.34) (end 165.1 55.88) (width 0.2) (layer "F.Cu") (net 5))
 (segment (start 157.48 60.96) (end 157.48 71.12) (width 0.2) (layer "F.Cu") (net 5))
 (segment (start 165.1 60.96) (end 157.48 60.96) (width 0.2) (layer "F.Cu") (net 5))
 (segment (start 149.86 78.74) (end 149.86 83.82) (width 0.2) (layer "F.Cu") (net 5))
 (segment (start 149.86 83.82) (end 144.78 83.82) (width 0.2) (layer "F.Cu") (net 5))
 (segment (start 157.48 71.12) (end 149.86 78.74) (width 0.2) (layer "F.Cu") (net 5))
 (segment (start 152.4 86.36) (end 144.78 86.36) (width 0.2) (layer "F.Cu") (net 6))
 (segment (start 157.48 73.66) (end 152.4 78.74) (width 0.2) (layer "F.Cu") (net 6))
 (segment (start 160.02 73.66) (end 157.48 73.66) (width 0.2) (layer "F.Cu") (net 6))
 (segment (start 160.06 66.04) (end 160.06 73.62) (width 0.2) (layer "F.Cu") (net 6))
 (segment (start 160.06 73.62) (end 160.02 73.66) (width 0.2) (layer "F.Cu") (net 6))
 (segment (start 152.4 78.74) (end 152.4 86.36) (width 0.2) (layer "F.Cu") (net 6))
 (segment (start 144.78 134.62) (end 139.7 129.54) (width 0.2) (layer "F.Cu") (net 23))
 (segment (start 132.08 129.54) (end 132.08 121.92) (width 0.2) (layer "F.Cu") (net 23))
 (segment (start 149.9 134.62) (end 144.78 134.62) (width 0.2) (layer "F.Cu") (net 23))
 (segment (start 139.7 129.54) (end 132.08 129.54) (width 0.2) (layer "F.Cu") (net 23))
 (segment (start 132.08 121.92) (end 130.69 121.92) (width 0.2) (layer "F.Cu") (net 23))
 (segment (start 130.742081 119.38) (end 129.54 119.38) (width 0.2) (layer "F.Cu") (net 26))
 (segment (start 162.56 127) (end 134.62 127) (width 0.2) (layer "F.Cu") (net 26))
 (segment (start 134.62 127) (end 134.62 123.257919) (width 0.2) (layer "F.Cu") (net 26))
 (segment (start 134.62 123.257919) (end 130.742081 119.38) (width 0.2) (layer "F.Cu") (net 26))
 (segment (start 162.56 132.12) (end 162.56 127) (width 0.2) (layer "F.Cu") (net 26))
 (segment (start 154.94 68.58) (end 149.86 73.66) (width 0.2) (layer "F.Cu") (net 4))
 (segment (start 147.32 78.74) (end 147.32 81.28) (width 0.2) (layer "F.Cu") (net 4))
 (segment (start 149.86 73.66) (end 149.86 76.2) (width 0.2) (layer "F.Cu") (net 4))
 (segment (start 157.52 53.34) (end 154.94 53.34) (width 0.2) (layer "F.Cu") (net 4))
 (segment (start 154.94 53.34) (end 154.94 68.58) (width 0.2) (layer "F.Cu") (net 4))
 (segment (start 149.86 76.2) (end 147.32 78.74) (width 0.2) (layer "F.Cu") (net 4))
 (segment (start 147.32 81.28) (end 144.78 81.28) (width 0.2) (layer "F.Cu") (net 4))
 (segment (start 154.94 78.74) (end 154.94 88.9) (width 0.2) (layer "F.Cu") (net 7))
 (segment (start 154.94 88.9) (end 144.78 88.9) (width 0.2) (layer "F.Cu") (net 7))
 (segment (start 156.795 78.74) (end 154.94 78.74) (width 0.2) (layer "F.Cu") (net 7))
 (segment (start 132.08 93.98) (end 129.54 93.98) (width 0.2) (layer "F.Cu") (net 21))
 (segment (start 137.56 78.34) (end 137.56 88.5) (width 0.2) (layer "F.Cu") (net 21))
 (segment (start 137.56 88.5) (end 132.08 93.98) (width 0.2) (layer "F.Cu") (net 21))
 (segment (start 142.24 73.66) (end 137.56 78.34) (width 0.2) (layer "F.Cu") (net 21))
 (segment (start 135.294814 57.745186) (end 132.08 67.80086) (width 0.2) (layer "F.Cu") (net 27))
 (segment (start 137.16 55.88) (end 135.294814 57.745186) (width 0.2) (layer "F.Cu") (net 27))
 (segment (start 132.08 67.80086) (end 132.08 81.28) (width 0.2) (layer "F.Cu") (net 27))
 (segment (start 132.08 81.28) (end 129.54 81.28) (width 0.2) (layer "F.Cu") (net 27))
 (segment (start 144.82 55.88) (end 137.16 55.88) (width 0.2) (layer "F.Cu") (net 27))
 (segment (start 139.7 78.74) (end 139.7 96.52) (width 0.2) (layer "F.Cu") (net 20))
 (segment (start 144.78 73.66) (end 139.7 78.74) (width 0.2) (layer "F.Cu") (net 20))
 (segment (start 139.7 96.52) (end 129.54 96.52) (width 0.2) (layer "F.Cu") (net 20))
 (segment (start 124.485 109.25) (end 121.95 109.25) (width 0.2) (layer "F.Cu") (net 24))
 (segment (start 121.95 109.25) (end 121.92 109.22) (width 0.2) (layer "F.Cu") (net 24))
 (segment (start 124.46 101.6) (end 129.54 101.6) (width 0.2) (layer "F.Cu") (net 24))
 (segment (start 121.92 104.14) (end 124.46 101.6) (width 0.2) (layer "F.Cu") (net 24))
 (segment (start 121.92 109.22) (end 121.92 104.14) (width 0.2) (layer "F.Cu") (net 24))
 (segment (start 119.38 107.525418) (end 120.970953 102.549047) (width 0.2) (layer "F.Cu") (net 25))
 (segment (start 120.970953 102.549047) (end 124.46 99.06) (width 0.2) (layer "F.Cu") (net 25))
 (segment (start 124.485 114.33) (end 121.95 114.33) (width 0.2) (layer "F.Cu") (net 25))
 (segment (start 119.38 109.22) (end 119.38 107.525418) (width 0.2) (layer "F.Cu") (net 25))
 (segment (start 121.92 114.3) (end 121.92 111.76) (width 0.2) (layer "F.Cu") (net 25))
 (segment (start 121.92 111.76) (end 119.38 109.22) (width 0.2) (layer "F.Cu") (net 25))
 (segment (start 121.95 114.33) (end 121.92 114.3) (width 0.2) (layer "F.Cu") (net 25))
 (segment (start 124.46 99.06) (end 129.54 99.06) (width 0.2) (layer "F.Cu") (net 25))
 (segment (start 167.68 99.06) (end 162.56 99.06) (width 0.2) (layer "F.Cu") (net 15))
 (segment (start 147.32 114.3) (end 144.78 114.3) (width 0.2) (layer "F.Cu") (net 15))
 (segment (start 147.32 111.76) (end 147.32 114.3) (width 0.2) (layer "F.Cu") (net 15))
 (segment (start 162.56 99.06) (end 149.86 111.76) (width 0.2) (layer "F.Cu") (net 15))
 (segment (start 149.86 111.76) (end 147.32 111.76) (width 0.2) (layer "F.Cu") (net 15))
 (segment (start 168.08 112.16) (end 152.4 112.16) (width 0.2) (layer "F.Cu") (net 16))
 (segment (start 152.4 112.16) (end 147.72 116.84) (width 0.2) (layer "F.Cu") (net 16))
 (segment (start 147.72 116.84) (end 144.78 116.84) (width 0.2) (layer "F.Cu") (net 16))
 (segment (start 172.76 116.84) (end 168.08 112.16) (width 0.2) (layer "F.Cu") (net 16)))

